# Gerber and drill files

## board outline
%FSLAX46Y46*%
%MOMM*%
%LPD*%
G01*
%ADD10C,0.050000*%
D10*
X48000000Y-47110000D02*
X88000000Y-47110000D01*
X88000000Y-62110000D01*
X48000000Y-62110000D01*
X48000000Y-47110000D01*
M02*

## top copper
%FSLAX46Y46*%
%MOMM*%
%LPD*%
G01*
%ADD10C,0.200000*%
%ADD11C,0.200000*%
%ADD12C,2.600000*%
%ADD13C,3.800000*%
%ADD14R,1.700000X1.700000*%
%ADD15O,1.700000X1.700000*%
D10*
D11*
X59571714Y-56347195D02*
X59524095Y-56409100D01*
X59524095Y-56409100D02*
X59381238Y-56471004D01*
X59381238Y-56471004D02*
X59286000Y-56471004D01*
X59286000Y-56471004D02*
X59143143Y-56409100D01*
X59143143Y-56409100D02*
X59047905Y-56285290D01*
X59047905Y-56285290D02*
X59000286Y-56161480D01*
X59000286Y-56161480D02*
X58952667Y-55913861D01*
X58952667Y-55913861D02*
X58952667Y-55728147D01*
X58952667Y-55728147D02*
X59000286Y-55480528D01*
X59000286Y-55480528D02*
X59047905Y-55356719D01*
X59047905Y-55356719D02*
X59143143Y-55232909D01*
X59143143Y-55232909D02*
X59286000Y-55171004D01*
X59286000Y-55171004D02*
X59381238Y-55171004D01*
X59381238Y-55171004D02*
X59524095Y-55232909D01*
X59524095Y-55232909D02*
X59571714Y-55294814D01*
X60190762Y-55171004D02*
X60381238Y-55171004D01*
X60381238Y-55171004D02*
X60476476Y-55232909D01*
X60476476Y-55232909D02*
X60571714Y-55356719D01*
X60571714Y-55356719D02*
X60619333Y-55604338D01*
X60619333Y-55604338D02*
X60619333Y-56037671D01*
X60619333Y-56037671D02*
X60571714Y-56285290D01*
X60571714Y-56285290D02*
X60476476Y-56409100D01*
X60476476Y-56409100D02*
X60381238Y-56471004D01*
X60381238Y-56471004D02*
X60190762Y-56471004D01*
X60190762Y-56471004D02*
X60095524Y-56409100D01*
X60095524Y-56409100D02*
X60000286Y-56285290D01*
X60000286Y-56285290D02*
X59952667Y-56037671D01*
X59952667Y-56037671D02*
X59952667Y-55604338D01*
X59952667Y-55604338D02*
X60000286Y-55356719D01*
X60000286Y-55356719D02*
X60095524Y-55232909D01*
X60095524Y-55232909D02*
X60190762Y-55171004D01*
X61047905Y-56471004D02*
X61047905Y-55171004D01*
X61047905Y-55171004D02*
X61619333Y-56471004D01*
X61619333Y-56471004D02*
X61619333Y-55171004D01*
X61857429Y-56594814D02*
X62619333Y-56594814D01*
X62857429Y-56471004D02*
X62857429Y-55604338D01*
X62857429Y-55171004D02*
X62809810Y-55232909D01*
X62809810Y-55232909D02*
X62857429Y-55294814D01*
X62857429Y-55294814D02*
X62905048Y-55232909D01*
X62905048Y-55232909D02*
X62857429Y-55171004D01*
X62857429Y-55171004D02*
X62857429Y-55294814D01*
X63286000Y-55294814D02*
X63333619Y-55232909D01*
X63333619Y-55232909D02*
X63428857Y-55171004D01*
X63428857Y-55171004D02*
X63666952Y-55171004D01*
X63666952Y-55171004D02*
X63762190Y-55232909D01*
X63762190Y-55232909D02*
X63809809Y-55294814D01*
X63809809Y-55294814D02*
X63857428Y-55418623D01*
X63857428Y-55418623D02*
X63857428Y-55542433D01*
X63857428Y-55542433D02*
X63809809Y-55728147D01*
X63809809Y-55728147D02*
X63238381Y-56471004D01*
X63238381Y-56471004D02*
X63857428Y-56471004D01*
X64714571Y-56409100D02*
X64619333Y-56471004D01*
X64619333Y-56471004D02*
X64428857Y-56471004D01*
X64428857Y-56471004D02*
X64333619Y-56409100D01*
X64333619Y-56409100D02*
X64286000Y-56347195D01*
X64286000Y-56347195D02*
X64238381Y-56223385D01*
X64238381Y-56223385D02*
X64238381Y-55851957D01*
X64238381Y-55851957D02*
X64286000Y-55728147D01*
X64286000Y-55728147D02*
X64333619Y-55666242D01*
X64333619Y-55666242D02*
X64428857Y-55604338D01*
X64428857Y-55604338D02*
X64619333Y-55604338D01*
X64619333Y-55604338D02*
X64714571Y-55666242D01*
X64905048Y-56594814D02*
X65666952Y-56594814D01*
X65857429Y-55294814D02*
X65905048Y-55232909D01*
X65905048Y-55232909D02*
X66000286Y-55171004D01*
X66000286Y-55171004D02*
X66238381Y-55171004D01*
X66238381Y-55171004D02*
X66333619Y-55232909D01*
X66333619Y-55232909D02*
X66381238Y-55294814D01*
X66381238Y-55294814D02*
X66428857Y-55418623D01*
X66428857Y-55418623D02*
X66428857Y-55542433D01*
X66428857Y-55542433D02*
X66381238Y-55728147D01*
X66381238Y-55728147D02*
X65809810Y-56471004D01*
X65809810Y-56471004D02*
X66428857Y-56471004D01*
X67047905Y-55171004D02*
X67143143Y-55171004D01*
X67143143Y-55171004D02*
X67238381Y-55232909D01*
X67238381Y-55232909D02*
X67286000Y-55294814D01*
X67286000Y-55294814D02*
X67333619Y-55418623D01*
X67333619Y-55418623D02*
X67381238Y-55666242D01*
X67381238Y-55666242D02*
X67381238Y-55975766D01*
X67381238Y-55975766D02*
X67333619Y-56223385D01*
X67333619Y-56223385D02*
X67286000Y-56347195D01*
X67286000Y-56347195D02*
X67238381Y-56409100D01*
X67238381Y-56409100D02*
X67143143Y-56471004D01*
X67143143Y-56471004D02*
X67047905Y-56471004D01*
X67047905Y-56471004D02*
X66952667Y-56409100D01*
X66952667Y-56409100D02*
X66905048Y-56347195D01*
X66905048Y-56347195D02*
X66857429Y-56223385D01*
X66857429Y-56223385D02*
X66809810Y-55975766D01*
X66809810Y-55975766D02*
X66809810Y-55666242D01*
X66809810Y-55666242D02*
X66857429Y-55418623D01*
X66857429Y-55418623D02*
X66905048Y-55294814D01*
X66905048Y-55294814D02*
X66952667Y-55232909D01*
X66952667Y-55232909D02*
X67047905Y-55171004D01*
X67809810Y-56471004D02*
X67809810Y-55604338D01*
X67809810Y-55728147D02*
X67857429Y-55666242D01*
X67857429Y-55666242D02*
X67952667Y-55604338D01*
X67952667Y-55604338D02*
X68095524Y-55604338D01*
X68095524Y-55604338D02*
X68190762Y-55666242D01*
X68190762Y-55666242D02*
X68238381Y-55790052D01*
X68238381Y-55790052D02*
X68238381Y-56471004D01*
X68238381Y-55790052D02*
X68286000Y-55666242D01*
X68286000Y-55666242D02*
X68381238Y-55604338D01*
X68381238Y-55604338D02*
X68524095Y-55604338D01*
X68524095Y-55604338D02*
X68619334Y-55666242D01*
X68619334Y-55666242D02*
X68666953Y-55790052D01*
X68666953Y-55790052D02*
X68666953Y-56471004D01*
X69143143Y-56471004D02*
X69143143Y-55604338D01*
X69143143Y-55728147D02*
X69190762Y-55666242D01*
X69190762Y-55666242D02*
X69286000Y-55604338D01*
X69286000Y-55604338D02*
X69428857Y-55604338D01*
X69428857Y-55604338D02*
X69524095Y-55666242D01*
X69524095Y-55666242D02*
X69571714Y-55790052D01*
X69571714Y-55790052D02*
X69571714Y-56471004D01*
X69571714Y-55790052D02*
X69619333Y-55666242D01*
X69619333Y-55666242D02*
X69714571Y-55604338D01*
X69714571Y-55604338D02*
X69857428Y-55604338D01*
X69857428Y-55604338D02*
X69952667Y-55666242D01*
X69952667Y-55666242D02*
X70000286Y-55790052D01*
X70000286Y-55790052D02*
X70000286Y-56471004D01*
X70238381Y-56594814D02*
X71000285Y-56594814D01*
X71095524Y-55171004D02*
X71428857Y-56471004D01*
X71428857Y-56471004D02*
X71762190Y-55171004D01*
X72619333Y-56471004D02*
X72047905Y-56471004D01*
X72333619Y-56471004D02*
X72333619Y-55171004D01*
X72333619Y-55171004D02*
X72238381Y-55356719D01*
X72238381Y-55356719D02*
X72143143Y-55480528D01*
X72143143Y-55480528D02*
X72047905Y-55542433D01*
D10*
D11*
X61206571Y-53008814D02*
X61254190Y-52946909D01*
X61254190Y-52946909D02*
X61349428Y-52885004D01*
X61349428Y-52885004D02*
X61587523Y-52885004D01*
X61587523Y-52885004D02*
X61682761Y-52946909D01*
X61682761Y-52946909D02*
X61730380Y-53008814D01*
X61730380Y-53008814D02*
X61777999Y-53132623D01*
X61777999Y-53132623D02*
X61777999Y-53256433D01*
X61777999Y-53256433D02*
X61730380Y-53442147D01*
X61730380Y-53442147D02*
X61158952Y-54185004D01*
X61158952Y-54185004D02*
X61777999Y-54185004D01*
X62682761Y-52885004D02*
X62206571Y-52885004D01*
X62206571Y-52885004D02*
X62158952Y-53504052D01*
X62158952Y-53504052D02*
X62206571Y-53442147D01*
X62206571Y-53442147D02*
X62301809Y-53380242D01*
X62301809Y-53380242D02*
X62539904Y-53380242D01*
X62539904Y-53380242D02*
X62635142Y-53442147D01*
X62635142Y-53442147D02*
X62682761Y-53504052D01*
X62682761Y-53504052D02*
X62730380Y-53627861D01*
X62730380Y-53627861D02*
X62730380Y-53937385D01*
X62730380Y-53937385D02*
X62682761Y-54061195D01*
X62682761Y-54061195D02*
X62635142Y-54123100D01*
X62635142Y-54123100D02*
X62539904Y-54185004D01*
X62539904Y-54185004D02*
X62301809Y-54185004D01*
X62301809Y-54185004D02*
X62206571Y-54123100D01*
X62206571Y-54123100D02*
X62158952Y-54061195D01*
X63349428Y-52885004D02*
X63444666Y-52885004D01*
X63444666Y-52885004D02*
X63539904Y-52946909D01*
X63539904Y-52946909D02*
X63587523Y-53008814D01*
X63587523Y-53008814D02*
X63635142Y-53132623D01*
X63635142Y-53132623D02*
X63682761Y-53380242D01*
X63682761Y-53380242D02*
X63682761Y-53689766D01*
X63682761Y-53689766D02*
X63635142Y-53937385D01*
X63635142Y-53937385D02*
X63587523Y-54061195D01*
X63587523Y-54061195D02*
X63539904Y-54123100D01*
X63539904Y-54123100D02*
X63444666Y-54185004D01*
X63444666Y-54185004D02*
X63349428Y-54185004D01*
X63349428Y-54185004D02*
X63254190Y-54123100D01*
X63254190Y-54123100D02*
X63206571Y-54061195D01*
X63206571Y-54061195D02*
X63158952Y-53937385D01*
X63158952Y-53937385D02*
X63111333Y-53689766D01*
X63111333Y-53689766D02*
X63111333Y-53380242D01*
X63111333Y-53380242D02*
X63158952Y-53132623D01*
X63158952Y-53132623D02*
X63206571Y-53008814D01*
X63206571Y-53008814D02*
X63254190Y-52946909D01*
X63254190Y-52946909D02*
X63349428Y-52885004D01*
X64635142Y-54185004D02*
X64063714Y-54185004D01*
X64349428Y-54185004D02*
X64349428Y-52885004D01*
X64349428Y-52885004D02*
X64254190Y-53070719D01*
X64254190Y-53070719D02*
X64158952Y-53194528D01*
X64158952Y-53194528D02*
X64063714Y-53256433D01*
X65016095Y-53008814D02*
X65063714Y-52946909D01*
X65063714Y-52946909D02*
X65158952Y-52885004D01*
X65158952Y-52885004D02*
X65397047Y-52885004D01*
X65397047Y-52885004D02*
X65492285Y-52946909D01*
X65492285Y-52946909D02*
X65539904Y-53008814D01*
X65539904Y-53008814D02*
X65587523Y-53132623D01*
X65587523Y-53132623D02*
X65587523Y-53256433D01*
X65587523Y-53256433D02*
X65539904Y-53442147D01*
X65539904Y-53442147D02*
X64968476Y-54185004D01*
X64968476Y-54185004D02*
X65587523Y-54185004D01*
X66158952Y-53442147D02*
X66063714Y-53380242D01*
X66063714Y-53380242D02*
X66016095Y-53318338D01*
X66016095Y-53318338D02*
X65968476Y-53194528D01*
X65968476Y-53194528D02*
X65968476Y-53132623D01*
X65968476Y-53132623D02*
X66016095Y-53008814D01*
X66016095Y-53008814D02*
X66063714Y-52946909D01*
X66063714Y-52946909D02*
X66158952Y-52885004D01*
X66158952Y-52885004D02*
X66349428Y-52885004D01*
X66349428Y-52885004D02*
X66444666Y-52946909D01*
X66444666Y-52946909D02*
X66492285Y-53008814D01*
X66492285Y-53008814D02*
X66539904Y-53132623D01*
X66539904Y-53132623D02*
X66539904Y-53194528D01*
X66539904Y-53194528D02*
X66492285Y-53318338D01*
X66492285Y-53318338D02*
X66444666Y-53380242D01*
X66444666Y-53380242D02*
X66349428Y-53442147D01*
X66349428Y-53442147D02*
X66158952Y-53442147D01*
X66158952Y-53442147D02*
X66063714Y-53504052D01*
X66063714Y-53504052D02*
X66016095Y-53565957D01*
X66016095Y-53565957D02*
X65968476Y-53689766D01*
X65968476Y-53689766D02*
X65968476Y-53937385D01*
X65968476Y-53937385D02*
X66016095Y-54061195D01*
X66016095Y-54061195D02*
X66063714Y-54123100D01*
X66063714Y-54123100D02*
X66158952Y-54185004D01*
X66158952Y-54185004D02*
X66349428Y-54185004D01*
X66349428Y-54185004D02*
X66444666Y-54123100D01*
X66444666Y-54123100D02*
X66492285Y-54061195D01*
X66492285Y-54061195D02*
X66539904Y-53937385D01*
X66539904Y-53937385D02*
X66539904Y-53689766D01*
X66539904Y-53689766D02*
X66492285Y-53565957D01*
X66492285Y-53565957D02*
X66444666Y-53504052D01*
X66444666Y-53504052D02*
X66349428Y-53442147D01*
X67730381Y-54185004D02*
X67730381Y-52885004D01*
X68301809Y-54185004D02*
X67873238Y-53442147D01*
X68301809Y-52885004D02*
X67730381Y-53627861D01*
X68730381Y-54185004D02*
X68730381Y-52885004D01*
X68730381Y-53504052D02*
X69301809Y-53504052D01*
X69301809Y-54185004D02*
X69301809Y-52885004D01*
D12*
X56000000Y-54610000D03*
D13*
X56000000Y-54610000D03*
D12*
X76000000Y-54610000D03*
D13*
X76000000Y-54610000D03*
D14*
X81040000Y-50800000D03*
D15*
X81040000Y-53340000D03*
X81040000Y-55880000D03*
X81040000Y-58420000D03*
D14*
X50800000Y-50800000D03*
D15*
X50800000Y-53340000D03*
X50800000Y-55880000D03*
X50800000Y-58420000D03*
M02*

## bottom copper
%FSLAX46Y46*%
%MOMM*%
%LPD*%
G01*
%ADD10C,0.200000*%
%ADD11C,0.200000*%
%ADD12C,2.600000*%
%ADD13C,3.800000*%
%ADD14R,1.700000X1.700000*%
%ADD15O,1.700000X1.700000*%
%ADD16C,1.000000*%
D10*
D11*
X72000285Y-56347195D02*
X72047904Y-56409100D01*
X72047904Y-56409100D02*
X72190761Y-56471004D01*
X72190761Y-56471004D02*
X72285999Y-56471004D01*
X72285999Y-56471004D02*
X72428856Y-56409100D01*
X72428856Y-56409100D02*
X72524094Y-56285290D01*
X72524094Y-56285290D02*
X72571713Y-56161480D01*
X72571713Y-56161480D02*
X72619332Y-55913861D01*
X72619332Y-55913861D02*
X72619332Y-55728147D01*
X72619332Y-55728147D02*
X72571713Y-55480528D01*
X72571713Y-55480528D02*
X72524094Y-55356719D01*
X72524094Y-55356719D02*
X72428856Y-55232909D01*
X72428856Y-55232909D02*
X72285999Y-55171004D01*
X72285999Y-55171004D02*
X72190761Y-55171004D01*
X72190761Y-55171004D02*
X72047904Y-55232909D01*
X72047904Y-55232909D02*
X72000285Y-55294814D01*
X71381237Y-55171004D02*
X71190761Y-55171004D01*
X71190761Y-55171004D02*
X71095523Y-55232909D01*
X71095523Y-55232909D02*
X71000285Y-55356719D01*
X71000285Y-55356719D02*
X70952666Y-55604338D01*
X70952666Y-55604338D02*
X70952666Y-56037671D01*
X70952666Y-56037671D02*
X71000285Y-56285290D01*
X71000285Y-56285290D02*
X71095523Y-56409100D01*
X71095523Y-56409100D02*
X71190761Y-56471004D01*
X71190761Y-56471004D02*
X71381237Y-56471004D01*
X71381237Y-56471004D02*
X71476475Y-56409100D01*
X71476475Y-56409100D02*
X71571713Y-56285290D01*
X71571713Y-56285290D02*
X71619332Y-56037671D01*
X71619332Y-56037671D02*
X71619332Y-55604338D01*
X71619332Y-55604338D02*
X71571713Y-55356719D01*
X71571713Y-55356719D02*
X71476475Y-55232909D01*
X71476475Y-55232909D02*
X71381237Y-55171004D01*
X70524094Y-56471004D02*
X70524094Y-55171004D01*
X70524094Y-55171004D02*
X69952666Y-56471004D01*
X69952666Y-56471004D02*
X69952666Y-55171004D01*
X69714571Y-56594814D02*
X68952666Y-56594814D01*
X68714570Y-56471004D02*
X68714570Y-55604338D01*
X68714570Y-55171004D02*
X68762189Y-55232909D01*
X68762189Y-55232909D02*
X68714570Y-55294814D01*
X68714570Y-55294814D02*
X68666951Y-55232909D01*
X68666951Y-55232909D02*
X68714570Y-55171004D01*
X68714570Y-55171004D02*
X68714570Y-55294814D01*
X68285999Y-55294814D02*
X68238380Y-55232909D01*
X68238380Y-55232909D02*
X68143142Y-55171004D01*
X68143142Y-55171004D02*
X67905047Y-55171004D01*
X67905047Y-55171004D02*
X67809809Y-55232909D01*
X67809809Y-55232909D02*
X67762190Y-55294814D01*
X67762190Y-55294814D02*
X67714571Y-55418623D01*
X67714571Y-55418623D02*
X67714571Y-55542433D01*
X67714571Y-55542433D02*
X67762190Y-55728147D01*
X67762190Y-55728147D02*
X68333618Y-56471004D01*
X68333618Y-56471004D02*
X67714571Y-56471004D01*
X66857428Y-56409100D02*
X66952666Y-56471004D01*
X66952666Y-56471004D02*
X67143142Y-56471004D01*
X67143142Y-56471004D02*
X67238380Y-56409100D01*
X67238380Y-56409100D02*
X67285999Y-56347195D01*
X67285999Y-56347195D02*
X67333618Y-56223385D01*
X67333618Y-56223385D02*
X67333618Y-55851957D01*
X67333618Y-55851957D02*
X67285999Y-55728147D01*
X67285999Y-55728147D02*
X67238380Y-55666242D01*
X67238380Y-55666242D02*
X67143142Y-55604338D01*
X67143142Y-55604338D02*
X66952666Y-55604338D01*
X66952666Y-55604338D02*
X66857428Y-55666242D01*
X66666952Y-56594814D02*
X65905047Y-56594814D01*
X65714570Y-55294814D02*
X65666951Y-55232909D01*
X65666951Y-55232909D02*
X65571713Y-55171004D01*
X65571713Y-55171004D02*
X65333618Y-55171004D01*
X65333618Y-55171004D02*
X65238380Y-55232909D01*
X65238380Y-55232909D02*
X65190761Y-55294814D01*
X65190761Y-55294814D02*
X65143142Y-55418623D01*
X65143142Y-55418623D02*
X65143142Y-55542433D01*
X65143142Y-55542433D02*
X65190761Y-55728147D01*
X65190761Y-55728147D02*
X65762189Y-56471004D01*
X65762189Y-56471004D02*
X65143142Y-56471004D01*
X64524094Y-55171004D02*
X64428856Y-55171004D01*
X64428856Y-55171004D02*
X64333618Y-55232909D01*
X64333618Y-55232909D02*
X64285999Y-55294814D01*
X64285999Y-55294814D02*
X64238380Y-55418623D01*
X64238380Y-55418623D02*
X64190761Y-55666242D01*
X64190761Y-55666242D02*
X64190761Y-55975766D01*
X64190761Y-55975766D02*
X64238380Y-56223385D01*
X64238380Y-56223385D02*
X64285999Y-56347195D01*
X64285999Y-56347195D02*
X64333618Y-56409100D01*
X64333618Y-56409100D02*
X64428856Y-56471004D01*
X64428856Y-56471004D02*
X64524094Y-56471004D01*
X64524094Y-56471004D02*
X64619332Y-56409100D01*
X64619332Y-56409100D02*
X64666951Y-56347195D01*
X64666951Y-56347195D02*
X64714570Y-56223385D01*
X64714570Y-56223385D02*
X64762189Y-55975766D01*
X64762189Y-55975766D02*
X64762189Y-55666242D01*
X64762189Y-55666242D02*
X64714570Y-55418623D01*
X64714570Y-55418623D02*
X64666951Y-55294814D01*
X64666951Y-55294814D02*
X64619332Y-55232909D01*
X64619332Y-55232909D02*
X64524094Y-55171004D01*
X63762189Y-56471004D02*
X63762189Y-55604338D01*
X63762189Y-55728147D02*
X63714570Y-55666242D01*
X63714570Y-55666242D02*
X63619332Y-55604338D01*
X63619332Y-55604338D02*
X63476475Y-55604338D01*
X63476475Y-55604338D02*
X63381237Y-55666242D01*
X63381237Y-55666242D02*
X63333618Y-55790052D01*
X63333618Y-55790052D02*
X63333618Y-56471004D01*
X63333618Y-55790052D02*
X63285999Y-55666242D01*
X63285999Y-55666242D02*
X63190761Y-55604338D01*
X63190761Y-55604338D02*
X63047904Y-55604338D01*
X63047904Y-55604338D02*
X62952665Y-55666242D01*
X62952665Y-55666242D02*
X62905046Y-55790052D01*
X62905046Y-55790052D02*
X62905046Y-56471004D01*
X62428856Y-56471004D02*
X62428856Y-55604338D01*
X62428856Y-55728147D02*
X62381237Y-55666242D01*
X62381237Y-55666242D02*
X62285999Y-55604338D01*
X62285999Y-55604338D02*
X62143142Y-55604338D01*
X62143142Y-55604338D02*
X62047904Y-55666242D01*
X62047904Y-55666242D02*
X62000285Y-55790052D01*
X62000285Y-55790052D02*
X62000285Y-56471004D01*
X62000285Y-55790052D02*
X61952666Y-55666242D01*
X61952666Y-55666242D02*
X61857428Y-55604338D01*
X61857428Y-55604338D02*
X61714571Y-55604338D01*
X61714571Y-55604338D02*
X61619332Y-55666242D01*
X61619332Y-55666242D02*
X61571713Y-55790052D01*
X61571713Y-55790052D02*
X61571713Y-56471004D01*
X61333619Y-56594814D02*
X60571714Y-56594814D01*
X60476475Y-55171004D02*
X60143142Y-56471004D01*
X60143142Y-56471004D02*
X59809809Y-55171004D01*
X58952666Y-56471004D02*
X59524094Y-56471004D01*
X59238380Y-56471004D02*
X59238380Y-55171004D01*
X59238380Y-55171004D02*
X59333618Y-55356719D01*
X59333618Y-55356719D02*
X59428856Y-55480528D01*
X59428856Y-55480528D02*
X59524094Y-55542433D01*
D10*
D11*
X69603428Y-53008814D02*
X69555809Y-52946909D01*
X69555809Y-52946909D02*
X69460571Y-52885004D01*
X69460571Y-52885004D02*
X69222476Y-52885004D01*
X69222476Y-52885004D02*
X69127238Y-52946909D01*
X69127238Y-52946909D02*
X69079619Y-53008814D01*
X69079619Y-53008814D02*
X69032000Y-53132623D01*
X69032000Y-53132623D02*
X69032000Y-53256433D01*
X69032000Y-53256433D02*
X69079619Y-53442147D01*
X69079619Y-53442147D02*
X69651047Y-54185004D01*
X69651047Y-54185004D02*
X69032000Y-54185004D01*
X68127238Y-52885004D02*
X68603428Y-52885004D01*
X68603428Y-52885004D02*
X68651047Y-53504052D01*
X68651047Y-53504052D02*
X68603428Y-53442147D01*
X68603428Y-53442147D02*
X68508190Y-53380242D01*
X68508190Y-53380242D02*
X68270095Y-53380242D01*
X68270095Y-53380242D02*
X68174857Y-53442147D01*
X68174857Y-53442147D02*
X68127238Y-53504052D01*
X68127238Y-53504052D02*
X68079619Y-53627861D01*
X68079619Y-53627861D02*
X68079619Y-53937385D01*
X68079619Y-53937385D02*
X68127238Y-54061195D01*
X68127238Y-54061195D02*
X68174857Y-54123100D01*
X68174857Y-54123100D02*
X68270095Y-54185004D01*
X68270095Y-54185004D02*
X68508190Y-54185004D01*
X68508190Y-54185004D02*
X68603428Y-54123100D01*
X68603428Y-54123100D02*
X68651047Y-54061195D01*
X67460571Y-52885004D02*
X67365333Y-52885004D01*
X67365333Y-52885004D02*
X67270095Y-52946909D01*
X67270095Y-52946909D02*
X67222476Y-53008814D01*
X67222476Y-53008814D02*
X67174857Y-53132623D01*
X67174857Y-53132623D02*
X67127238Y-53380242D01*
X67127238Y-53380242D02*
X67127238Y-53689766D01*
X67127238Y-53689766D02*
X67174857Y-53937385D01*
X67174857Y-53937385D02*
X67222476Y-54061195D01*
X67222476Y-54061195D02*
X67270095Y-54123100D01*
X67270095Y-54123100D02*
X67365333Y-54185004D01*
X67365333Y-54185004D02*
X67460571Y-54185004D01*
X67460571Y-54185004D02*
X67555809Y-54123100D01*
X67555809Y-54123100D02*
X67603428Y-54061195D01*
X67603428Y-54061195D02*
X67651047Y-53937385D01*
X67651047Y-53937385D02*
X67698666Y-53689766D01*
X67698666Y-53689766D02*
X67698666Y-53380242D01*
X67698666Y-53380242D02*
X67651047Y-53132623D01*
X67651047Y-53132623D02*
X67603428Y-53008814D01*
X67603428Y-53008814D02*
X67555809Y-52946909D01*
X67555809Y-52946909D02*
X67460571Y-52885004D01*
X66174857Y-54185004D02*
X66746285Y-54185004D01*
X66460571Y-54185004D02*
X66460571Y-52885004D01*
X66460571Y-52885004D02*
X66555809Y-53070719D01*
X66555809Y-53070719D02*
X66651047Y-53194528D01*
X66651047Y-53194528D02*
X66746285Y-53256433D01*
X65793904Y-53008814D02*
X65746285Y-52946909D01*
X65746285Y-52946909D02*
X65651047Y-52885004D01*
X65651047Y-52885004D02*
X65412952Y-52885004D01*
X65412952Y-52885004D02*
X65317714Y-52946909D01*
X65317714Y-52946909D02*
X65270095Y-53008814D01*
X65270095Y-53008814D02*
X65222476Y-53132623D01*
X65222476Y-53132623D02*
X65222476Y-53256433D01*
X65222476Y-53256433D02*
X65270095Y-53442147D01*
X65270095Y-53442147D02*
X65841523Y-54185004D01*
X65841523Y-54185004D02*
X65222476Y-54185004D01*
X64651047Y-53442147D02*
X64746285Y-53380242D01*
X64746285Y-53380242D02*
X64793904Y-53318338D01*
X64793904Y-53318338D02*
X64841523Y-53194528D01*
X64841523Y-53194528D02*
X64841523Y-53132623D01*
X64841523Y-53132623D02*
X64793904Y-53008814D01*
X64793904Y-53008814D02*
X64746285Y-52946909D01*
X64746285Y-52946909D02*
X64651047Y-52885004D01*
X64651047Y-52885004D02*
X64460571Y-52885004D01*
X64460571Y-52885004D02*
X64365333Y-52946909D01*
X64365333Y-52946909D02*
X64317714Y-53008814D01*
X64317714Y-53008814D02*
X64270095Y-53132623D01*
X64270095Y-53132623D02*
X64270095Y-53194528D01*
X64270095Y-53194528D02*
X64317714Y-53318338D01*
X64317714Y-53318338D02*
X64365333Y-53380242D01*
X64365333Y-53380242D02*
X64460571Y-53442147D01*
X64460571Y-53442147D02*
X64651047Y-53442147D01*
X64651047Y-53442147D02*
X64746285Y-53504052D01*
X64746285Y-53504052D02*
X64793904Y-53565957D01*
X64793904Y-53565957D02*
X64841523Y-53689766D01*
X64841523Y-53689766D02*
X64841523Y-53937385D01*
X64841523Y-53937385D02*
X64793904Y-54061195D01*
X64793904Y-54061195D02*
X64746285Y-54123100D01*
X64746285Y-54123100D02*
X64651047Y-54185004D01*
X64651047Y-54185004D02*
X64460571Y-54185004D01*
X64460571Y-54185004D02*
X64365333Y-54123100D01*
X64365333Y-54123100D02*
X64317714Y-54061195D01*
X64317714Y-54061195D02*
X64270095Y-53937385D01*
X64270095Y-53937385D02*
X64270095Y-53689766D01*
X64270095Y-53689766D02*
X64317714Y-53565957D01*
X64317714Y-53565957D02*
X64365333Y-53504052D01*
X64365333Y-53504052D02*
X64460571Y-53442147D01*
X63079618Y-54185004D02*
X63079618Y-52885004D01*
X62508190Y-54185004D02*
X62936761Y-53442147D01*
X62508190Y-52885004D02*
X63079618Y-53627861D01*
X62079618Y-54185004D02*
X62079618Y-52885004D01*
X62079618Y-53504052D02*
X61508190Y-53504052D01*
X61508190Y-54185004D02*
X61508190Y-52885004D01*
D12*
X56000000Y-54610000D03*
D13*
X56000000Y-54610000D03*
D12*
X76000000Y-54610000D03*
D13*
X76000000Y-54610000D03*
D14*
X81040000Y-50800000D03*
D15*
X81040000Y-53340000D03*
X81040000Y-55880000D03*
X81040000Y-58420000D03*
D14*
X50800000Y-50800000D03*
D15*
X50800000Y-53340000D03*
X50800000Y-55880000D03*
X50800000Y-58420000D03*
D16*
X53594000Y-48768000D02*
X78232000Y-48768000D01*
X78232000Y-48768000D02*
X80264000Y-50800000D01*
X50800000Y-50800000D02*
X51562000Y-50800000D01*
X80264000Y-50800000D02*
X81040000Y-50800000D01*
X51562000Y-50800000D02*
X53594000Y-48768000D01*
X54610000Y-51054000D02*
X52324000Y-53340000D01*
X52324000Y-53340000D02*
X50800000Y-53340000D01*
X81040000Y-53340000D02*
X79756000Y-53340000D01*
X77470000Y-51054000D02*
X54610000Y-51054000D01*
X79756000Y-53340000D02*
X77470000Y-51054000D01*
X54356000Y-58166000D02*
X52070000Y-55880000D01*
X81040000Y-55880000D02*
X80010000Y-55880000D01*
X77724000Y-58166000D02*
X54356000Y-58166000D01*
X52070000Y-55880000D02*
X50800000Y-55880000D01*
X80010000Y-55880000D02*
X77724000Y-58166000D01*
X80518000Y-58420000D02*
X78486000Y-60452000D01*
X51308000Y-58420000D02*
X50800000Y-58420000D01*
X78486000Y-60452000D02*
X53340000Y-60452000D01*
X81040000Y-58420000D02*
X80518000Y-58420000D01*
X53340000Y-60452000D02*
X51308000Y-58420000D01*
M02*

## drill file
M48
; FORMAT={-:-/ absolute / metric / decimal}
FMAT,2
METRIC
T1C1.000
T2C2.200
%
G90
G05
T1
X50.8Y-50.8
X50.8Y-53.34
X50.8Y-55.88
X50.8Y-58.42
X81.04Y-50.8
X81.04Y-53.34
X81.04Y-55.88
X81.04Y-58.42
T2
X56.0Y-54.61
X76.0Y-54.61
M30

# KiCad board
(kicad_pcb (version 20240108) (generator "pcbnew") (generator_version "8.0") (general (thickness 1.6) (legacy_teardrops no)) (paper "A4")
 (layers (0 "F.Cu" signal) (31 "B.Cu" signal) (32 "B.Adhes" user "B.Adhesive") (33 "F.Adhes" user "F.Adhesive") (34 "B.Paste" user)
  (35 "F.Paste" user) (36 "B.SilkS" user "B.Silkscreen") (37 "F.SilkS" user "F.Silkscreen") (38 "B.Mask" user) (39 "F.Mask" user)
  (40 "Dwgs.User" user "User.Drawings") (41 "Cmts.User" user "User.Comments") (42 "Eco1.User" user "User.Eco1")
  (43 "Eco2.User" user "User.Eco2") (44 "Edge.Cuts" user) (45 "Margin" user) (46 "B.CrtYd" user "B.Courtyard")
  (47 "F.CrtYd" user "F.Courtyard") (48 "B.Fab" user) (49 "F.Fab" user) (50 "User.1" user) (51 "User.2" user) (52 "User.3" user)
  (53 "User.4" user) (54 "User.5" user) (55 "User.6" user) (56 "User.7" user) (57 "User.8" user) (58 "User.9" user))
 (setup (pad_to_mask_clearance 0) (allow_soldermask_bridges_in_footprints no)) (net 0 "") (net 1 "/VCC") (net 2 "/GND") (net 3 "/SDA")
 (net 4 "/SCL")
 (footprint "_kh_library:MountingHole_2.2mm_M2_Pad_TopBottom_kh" (layer "F.Cu") (at 56 54.61)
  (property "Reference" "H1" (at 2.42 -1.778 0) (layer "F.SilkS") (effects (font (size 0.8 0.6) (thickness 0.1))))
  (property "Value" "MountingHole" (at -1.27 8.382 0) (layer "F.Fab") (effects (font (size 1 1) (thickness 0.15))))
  (pad "1" thru_hole circle (at 0 0) (size 2.6 2.6) (drill 2.2) (layers "*.Cu" "*.Mask") (remove_unused_layers no))
  (pad "1" connect circle (at 0 0) (size 3.8 3.8) (layers "F.Cu" "F.Mask"))
  (pad "1" connect circle (at 0 0) (size 3.8 3.8) (layers "B.Cu" "B.Mask")))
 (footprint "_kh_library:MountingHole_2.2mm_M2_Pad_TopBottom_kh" (layer "F.Cu") (at 76 54.61)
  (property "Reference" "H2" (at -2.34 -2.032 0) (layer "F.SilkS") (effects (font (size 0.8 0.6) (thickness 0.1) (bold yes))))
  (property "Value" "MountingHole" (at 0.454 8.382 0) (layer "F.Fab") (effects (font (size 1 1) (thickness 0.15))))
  (pad "1" thru_hole circle (at 0 0) (size 2.6 2.6) (drill 2.2) (layers "*.Cu" "*.Mask") (remove_unused_layers no))
  (pad "1" connect circle (at 0 0) (size 3.8 3.8) (layers "F.Cu" "F.Mask"))
  (pad "1" connect circle (at 0 0) (size 3.8 3.8) (layers "B.Cu" "B.Mask")))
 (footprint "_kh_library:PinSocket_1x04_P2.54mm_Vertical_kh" (layer "F.Cu") (at 81.04 50.8)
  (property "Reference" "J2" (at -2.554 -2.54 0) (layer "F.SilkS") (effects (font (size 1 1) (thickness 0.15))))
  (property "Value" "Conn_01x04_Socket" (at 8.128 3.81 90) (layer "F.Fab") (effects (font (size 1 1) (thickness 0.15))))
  (pad "1" thru_hole rect (at 0 0) (size 1.7 1.7) (drill 1) (layers "*.Cu" "*.Mask") (remove_unused_layers no) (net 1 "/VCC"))
  (pad "2" thru_hole oval (at 0 2.54) (size 1.7 1.7) (drill 1) (layers "*.Cu" "*.Mask") (remove_unused_layers no) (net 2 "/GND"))
  (pad "3" thru_hole oval (at 0 5.08) (size 1.7 1.7) (drill 1) (layers "*.Cu" "*.Mask") (remove_unused_layers no) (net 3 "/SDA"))
  (pad "4" thru_hole oval (at 0 7.62) (size 1.7 1.7) (drill 1) (layers "*.Cu" "*.Mask") (remove_unused_layers no) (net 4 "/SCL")))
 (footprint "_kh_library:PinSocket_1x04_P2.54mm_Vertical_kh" (layer "F.Cu") (at 50.8 50.8)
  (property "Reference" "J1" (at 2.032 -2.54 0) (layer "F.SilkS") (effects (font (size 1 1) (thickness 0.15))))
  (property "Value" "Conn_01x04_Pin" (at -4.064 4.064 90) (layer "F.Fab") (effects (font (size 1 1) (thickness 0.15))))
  (pad "1" thru_hole rect (at 0 0) (size 1.7 1.7) (drill 1) (layers "*.Cu" "*.Mask") (remove_unused_layers no) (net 1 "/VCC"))
  (pad "2" thru_hole oval (at 0 2.54) (size 1.7 1.7) (drill 1) (layers "*.Cu" "*.Mask") (remove_unused_layers no) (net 2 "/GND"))
  (pad "3" thru_hole oval (at 0 5.08) (size 1.7 1.7) (drill 1) (layers "*.Cu" "*.Mask") (remove_unused_layers no) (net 3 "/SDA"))
  (pad "4" thru_hole oval (at 0 7.62) (size 1.7 1.7) (drill 1) (layers "*.Cu" "*.Mask") (remove_unused_layers no) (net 4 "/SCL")))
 (gr_rect (start 48 47.11) (end 88 62.11) (stroke (width 0.05) (type default)) (fill none) (layer "Edge.Cuts"))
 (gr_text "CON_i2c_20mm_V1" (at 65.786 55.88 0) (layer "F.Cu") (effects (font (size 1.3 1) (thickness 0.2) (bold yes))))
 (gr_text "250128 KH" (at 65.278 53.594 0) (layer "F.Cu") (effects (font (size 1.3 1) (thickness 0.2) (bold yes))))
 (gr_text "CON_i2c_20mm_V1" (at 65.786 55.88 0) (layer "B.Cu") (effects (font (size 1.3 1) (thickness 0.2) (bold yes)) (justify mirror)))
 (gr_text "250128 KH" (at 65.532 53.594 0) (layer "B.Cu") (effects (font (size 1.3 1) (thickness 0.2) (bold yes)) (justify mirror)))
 (segment (start 53.594 48.768) (end 78.232 48.768) (width 1) (layer "B.Cu") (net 1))
 (segment (start 78.232 48.768) (end 80.264 50.8) (width 1) (layer "B.Cu") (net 1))
 (segment (start 50.8 50.8) (end 51.562 50.8) (width 1) (layer "B.Cu") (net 1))
 (segment (start 80.264 50.8) (end 81.04 50.8) (width 1) (layer "B.Cu") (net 1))
 (segment (start 51.562 50.8) (end 53.594 48.768) (width 1) (layer "B.Cu") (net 1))
 (segment (start 54.61 51.054) (end 52.324 53.34) (width 1) (layer "B.Cu") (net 2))
 (segment (start 52.324 53.34) (end 50.8 53.34) (width 1) (layer "B.Cu") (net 2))
 (segment (start 81.04 53.34) (end 79.756 53.34) (width 1) (layer "B.Cu") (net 2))
 (segment (start 77.47 51.054) (end 54.61 51.054) (width 1) (layer "B.Cu") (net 2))
 (segment (start 79.756 53.34) (end 77.47 51.054) (width 1) (layer "B.Cu") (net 2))
 (segment (start 54.356 58.166) (end 52.07 55.88) (width 1) (layer "B.Cu") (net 3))
 (segment (start 81.04 55.88) (end 80.01 55.88) (width 1) (layer "B.Cu") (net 3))
 (segment (start 77.724 58.166) (end 54.356 58.166) (width 1) (layer "B.Cu") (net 3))
 (segment (start 52.07 55.88) (end 50.8 55.88) (width 1) (layer "B.Cu") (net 3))
 (segment (start 80.01 55.88) (end 77.724 58.166) (width 1) (layer "B.Cu") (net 3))
 (segment (start 80.518 58.42) (end 78.486 60.452) (width 1) (layer "B.Cu") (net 4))
 (segment (start 51.308 58.42) (end 50.8 58.42) (width 1) (layer "B.Cu") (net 4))
 (segment (start 78.486 60.452) (end 53.34 60.452) (width 1) (layer "B.Cu") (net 4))
 (segment (start 81.04 58.42) (end 80.518 58.42) (width 1) (layer "B.Cu") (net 4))
 (segment (start 53.34 60.452) (end 51.308 58.42) (width 1) (layer "B.Cu") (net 4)))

